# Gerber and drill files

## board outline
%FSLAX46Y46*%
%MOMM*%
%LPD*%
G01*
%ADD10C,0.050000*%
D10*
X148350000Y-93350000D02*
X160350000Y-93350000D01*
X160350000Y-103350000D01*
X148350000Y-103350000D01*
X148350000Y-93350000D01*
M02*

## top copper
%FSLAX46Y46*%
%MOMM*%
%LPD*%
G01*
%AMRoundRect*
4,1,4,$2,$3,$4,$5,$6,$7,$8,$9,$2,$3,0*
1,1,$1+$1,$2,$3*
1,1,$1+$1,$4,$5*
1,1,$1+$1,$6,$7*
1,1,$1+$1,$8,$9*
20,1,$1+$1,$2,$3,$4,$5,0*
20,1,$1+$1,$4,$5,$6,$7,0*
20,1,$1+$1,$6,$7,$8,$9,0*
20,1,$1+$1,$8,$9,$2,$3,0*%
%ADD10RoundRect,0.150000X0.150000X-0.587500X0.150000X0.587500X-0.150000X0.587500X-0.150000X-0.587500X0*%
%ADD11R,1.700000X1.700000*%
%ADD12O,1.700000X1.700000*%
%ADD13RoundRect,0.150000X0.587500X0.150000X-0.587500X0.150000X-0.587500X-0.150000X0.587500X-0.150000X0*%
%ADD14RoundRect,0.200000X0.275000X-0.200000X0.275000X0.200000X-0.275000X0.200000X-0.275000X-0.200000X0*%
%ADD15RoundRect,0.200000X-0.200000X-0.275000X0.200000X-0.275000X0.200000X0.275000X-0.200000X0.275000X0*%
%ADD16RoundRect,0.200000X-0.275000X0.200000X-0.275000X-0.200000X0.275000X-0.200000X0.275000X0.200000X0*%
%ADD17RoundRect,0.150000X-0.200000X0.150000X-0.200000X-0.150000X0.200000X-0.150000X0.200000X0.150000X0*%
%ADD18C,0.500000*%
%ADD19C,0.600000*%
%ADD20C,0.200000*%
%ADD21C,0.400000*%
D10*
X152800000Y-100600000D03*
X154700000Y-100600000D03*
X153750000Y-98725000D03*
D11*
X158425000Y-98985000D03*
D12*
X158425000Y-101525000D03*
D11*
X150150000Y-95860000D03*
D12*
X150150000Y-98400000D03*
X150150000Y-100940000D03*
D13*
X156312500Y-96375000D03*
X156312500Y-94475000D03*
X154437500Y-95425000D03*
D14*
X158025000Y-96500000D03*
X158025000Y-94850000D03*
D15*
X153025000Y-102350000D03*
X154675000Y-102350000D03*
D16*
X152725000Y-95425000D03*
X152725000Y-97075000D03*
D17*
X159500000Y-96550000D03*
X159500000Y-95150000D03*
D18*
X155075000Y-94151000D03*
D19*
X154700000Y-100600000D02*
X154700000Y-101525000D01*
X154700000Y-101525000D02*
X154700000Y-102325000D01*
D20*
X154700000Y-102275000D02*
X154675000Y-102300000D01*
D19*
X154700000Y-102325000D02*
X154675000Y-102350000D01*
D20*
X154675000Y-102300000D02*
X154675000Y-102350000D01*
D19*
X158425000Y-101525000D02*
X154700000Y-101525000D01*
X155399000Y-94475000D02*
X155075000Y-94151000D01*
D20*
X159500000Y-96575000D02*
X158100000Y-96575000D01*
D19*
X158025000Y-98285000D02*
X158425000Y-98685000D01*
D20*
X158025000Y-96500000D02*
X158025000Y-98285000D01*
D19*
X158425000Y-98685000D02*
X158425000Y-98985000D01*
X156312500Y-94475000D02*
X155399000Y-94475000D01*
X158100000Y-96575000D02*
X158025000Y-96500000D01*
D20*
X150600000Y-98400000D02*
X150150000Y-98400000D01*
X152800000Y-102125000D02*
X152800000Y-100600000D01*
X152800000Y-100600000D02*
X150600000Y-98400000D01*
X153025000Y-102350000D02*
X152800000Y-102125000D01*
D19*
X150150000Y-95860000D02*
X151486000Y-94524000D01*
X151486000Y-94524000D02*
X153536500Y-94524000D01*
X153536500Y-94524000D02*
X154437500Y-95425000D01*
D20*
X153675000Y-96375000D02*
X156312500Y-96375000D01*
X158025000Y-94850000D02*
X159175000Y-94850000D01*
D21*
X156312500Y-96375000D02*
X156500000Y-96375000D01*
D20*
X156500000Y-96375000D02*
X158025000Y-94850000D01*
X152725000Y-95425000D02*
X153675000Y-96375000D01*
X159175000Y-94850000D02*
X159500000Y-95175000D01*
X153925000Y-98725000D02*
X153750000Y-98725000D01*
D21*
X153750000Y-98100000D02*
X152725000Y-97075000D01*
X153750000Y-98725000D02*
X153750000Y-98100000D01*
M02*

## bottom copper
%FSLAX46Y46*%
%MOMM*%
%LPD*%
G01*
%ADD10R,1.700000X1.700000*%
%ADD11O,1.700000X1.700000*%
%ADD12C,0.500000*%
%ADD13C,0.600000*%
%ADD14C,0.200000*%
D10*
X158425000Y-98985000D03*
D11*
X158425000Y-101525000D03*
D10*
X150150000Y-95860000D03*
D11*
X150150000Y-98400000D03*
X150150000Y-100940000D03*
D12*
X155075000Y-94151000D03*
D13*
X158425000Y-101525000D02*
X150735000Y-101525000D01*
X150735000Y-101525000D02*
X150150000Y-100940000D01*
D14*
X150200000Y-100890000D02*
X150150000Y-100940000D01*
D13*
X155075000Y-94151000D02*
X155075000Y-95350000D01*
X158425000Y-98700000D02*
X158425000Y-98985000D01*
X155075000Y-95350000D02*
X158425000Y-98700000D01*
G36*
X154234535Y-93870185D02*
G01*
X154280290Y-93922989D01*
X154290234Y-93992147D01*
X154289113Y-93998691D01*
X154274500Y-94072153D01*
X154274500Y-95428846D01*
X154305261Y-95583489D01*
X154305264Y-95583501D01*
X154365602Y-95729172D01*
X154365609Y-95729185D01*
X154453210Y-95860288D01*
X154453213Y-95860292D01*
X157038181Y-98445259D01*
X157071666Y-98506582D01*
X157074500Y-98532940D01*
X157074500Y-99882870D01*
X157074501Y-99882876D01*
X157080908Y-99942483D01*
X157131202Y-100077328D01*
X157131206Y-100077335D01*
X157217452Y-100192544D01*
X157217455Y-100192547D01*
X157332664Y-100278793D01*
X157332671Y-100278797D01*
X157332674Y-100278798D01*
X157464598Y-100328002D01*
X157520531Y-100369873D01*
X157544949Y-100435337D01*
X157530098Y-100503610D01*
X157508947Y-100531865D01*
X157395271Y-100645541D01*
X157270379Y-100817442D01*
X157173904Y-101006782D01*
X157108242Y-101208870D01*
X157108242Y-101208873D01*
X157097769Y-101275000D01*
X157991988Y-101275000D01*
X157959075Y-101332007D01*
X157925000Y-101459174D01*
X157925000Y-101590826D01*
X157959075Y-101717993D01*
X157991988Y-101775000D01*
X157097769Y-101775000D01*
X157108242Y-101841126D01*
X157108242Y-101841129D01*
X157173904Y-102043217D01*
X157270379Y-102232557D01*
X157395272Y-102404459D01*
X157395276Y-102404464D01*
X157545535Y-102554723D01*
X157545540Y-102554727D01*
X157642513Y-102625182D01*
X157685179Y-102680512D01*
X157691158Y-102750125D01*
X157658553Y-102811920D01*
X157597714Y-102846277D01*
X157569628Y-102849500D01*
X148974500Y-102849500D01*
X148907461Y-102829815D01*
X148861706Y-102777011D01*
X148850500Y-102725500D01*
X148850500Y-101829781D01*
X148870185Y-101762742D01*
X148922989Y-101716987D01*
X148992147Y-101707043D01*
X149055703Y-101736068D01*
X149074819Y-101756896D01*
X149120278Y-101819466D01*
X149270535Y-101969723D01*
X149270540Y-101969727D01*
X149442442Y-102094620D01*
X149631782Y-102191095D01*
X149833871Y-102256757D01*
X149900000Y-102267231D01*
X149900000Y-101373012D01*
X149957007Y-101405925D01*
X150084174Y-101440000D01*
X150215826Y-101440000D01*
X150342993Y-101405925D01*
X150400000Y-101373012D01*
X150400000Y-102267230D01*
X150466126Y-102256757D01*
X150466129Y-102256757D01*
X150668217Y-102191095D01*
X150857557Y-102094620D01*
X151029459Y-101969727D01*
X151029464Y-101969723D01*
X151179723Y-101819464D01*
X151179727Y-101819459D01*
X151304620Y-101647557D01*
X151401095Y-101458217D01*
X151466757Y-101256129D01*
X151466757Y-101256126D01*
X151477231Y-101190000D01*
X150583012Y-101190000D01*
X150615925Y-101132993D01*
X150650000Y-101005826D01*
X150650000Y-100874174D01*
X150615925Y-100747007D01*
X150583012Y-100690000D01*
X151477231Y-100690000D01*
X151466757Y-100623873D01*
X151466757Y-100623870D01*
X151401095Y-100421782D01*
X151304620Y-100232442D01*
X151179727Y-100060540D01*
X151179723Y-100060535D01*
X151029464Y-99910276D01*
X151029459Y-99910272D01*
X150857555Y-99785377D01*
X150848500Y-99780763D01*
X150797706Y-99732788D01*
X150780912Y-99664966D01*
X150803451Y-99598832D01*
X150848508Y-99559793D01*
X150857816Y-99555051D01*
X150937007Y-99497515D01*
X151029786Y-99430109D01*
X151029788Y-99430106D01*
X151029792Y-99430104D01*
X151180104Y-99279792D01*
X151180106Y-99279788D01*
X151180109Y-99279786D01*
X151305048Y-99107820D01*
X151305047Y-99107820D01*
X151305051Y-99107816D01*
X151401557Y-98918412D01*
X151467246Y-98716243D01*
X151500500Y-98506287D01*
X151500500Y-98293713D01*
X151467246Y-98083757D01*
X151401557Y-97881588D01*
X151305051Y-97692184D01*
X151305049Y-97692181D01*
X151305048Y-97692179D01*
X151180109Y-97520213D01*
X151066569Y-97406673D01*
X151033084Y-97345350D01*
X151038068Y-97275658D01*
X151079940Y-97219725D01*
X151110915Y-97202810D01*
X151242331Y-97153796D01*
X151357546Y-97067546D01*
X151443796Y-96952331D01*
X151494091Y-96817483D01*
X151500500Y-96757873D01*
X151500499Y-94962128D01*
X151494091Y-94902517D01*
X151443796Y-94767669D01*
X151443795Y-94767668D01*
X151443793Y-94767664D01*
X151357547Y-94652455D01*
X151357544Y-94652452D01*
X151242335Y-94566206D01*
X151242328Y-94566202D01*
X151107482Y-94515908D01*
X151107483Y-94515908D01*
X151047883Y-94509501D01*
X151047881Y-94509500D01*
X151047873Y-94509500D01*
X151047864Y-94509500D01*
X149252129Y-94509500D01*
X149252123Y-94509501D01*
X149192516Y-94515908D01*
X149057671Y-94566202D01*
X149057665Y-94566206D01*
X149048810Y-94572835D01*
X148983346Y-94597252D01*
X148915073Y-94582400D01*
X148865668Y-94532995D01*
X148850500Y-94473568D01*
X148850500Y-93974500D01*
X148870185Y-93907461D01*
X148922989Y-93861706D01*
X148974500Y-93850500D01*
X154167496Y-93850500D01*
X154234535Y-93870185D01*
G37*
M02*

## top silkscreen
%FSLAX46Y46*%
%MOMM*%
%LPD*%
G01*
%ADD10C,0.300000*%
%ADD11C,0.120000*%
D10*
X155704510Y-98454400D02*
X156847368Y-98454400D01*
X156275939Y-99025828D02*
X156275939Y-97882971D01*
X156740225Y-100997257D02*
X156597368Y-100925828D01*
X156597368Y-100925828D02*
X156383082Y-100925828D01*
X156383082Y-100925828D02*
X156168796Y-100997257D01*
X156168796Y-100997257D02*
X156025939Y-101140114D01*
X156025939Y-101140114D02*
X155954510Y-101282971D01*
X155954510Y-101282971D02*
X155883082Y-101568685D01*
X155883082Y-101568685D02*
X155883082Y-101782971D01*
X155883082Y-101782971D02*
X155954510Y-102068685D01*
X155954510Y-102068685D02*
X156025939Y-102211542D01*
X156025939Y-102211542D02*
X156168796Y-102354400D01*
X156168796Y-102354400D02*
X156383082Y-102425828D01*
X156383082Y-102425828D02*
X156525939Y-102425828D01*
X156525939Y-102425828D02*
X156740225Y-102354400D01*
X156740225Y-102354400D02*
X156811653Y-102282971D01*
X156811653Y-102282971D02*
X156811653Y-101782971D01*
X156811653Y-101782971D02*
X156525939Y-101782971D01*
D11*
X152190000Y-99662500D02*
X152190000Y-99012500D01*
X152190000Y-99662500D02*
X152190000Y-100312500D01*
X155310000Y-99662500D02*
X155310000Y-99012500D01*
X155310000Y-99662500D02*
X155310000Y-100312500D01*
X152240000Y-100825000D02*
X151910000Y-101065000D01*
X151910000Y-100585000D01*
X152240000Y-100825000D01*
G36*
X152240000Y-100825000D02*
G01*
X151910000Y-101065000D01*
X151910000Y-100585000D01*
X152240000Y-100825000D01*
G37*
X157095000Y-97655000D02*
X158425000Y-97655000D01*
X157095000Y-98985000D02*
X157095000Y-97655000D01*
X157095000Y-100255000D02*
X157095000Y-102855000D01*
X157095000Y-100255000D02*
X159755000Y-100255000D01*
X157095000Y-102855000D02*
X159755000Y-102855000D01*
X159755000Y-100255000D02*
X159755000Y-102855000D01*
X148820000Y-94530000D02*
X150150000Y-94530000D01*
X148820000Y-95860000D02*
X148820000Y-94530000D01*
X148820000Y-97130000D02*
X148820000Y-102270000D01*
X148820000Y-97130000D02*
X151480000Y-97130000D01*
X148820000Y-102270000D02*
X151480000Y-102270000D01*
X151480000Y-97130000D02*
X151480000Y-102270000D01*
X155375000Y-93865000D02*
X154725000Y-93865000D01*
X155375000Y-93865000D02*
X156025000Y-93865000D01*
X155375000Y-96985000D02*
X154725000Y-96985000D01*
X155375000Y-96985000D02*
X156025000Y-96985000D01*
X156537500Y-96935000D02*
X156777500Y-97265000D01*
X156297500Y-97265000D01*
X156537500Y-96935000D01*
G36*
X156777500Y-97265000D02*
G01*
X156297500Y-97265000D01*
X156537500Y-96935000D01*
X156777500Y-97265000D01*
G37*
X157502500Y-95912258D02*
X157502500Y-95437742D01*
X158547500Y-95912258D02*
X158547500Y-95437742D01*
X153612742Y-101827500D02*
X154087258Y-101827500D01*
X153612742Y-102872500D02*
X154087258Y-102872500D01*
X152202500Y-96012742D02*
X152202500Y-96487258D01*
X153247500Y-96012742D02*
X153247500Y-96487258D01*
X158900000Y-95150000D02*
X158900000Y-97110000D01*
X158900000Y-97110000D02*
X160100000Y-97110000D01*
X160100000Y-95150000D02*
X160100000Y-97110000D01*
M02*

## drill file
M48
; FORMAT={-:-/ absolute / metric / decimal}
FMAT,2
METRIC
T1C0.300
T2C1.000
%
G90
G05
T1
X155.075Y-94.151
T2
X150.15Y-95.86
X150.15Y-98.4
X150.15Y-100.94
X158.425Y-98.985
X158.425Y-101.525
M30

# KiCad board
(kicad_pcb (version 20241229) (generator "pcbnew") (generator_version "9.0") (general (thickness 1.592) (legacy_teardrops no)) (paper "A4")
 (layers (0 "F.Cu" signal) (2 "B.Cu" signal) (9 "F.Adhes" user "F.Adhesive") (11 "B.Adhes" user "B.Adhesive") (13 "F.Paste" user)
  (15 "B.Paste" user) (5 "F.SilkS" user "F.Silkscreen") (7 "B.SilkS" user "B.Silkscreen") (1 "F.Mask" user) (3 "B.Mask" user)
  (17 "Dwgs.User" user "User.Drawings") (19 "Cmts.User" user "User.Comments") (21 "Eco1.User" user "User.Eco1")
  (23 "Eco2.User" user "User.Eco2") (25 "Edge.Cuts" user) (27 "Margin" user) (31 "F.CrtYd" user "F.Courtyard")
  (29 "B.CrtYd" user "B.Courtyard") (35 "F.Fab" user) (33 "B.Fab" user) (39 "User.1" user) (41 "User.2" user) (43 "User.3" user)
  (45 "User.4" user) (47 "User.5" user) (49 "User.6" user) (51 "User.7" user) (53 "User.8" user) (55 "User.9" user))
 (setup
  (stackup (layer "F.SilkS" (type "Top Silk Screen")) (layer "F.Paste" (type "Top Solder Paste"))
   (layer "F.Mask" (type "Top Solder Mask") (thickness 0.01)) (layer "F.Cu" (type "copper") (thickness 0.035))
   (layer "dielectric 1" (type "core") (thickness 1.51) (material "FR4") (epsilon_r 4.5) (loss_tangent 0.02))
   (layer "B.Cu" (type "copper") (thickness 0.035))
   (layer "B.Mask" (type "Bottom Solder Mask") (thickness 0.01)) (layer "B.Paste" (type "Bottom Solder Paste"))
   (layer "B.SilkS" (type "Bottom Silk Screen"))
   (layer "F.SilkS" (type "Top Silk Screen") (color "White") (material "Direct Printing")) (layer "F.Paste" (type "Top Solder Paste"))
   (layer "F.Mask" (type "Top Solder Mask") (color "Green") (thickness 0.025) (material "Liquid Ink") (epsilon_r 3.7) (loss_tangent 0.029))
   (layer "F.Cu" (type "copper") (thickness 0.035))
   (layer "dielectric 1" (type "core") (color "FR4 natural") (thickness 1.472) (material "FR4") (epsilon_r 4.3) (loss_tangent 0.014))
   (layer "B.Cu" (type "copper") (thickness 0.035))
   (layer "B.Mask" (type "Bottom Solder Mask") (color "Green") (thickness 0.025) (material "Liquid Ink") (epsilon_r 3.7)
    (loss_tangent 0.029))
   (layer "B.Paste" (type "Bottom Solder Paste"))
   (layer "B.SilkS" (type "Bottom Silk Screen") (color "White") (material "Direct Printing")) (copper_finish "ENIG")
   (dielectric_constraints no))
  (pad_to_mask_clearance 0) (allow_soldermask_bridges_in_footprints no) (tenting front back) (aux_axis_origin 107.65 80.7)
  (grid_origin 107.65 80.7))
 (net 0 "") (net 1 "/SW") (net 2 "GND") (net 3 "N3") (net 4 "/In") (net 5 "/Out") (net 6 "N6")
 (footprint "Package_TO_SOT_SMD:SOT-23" (layer "F.Cu") (at 153.75 99.6625 90)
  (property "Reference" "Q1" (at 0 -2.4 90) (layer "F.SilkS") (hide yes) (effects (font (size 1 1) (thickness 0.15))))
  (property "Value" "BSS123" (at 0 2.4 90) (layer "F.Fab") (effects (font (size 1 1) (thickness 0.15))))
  (fp_line (start 0 -1.56) (end 0.65 -1.56) (stroke (width 0.12) (type solid)) (layer "F.SilkS"))
  (fp_line (start 0 -1.56) (end -0.65 -1.56) (stroke (width 0.12) (type solid)) (layer "F.SilkS"))
  (fp_line (start 0 1.56) (end 0.65 1.56) (stroke (width 0.12) (type solid)) (layer "F.SilkS"))
  (fp_line (start 0 1.56) (end -0.65 1.56) (stroke (width 0.12) (type solid)) (layer "F.SilkS"))
  (fp_poly
   (pts (xy -1.1625 -1.51) (xy -1.4025 -1.84) (xy -0.9225 -1.84) (xy -1.1625 -1.51)) (stroke (width 0.12) (type solid)) (fill yes)
   (layer "F.SilkS"))
  (pad "1" smd roundrect (at -0.9375 -0.95 90) (size 1.475 0.6) (layers "F.Cu" "F.Mask" "F.Paste") (roundrect_rratio 0.25) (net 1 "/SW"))
  (pad "2" smd roundrect (at -0.9375 0.95 90) (size 1.475 0.6) (layers "F.Cu" "F.Mask" "F.Paste") (roundrect_rratio 0.25) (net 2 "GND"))
  (pad "3" smd roundrect (at 0.9375 0 90) (size 1.475 0.6) (layers "F.Cu" "F.Mask" "F.Paste") (roundrect_rratio 0.25) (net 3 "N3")))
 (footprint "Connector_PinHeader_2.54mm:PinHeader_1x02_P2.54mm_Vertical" (layer "F.Cu") (at 158.425 98.985)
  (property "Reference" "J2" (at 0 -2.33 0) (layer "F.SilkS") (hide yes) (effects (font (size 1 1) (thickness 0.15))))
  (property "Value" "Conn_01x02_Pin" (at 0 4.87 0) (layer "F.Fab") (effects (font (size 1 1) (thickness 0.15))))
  (fp_line (start -1.33 -1.33) (end 0 -1.33) (stroke (width 0.12) (type solid)) (layer "F.SilkS"))
  (fp_line (start -1.33 0) (end -1.33 -1.33) (stroke (width 0.12) (type solid)) (layer "F.SilkS"))
  (fp_line (start -1.33 1.27) (end -1.33 3.87) (stroke (width 0.12) (type solid)) (layer "F.SilkS"))
  (fp_line (start -1.33 1.27) (end 1.33 1.27) (stroke (width 0.12) (type solid)) (layer "F.SilkS"))
  (fp_line (start -1.33 3.87) (end 1.33 3.87) (stroke (width 0.12) (type solid)) (layer "F.SilkS"))
  (fp_line (start 1.33 1.27) (end 1.33 3.87) (stroke (width 0.12) (type solid)) (layer "F.SilkS"))
  (pad "1" thru_hole rect (at 0 0) (size 1.7 1.7) (drill 1) (layers "*.Cu" "*.Mask") (remove_unused_layers no) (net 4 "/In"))
  (pad "2" thru_hole oval (at 0 2.54) (size 1.7 1.7) (drill 1) (layers "*.Cu" "*.Mask") (remove_unused_layers no) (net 2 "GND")))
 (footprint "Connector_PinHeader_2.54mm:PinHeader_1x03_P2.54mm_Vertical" (layer "F.Cu") (at 150.15 95.86)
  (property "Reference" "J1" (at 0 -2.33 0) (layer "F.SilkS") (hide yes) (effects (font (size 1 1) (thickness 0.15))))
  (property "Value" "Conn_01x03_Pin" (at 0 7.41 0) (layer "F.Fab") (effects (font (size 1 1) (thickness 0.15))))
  (fp_line (start -1.33 -1.33) (end 0 -1.33) (stroke (width 0.12) (type solid)) (layer "F.SilkS"))
  (fp_line (start -1.33 0) (end -1.33 -1.33) (stroke (width 0.12) (type solid)) (layer "F.SilkS"))
  (fp_line (start -1.33 1.27) (end -1.33 6.41) (stroke (width 0.12) (type solid)) (layer "F.SilkS"))
  (fp_line (start -1.33 1.27) (end 1.33 1.27) (stroke (width 0.12) (type solid)) (layer "F.SilkS"))
  (fp_line (start -1.33 6.41) (end 1.33 6.41) (stroke (width 0.12) (type solid)) (layer "F.SilkS"))
  (fp_line (start 1.33 1.27) (end 1.33 6.41) (stroke (width 0.12) (type solid)) (layer "F.SilkS"))
  (pad "1" thru_hole rect (at 0 0) (size 1.7 1.7) (drill 1) (layers "*.Cu" "*.Mask") (remove_unused_layers no) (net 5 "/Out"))
  (pad "2" thru_hole oval (at 0 2.54) (size 1.7 1.7) (drill 1) (layers "*.Cu" "*.Mask") (remove_unused_layers no) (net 1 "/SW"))
  (pad "3" thru_hole oval (at 0 5.08) (size 1.7 1.7) (drill 1) (layers "*.Cu" "*.Mask") (remove_unused_layers no) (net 2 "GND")))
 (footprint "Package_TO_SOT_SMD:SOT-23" (layer "F.Cu") (at 155.375 95.425 180)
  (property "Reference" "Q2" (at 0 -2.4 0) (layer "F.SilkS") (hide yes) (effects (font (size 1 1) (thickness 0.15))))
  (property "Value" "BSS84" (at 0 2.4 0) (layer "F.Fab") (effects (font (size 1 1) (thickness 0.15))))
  (fp_line (start 0 1.56) (end 0.65 1.56) (stroke (width 0.12) (type solid)) (layer "F.SilkS"))
  (fp_line (start 0 1.56) (end -0.65 1.56) (stroke (width 0.12) (type solid)) (layer "F.SilkS"))
  (fp_line (start 0 -1.56) (end 0.65 -1.56) (stroke (width 0.12) (type solid)) (layer "F.SilkS"))
  (fp_line (start 0 -1.56) (end -0.65 -1.56) (stroke (width 0.12) (type solid)) (layer "F.SilkS"))
  (fp_poly
   (pts (xy -1.1625 -1.51) (xy -1.4025 -1.84) (xy -0.9225 -1.84) (xy -1.1625 -1.51)) (stroke (width 0.12) (type solid)) (fill yes)
   (layer "F.SilkS"))
  (pad "1" smd roundrect (at -0.9375 -0.95 180) (size 1.475 0.6) (layers "F.Cu" "F.Mask" "F.Paste") (roundrect_rratio 0.25) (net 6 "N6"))
  (pad "2" smd roundrect (at -0.9375 0.95 180) (size 1.475 0.6) (layers "F.Cu" "F.Mask" "F.Paste") (roundrect_rratio 0.25) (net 4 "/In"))
  (pad "3" smd roundrect (at 0.9375 0 180) (size 1.475 0.6) (layers "F.Cu" "F.Mask" "F.Paste") (roundrect_rratio 0.25) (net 5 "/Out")))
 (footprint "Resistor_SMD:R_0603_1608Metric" (layer "F.Cu") (at 158.025 95.675 90)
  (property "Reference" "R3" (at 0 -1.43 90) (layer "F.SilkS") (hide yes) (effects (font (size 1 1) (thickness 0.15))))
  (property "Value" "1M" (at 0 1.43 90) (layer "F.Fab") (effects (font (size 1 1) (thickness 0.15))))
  (fp_line (start -0.237258 -0.5225) (end 0.237258 -0.5225) (stroke (width 0.12) (type solid)) (layer "F.SilkS"))
  (fp_line (start -0.237258 0.5225) (end 0.237258 0.5225) (stroke (width 0.12) (type solid)) (layer "F.SilkS"))
  (pad "1" smd roundrect (at -0.825 0 90) (size 0.8 0.95) (layers "F.Cu" "F.Mask" "F.Paste") (roundrect_rratio 0.25) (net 4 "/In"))
  (pad "2" smd roundrect (at 0.825 0 90) (size 0.8 0.95) (layers "F.Cu" "F.Mask" "F.Paste") (roundrect_rratio 0.25) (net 6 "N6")))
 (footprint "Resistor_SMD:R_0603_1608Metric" (layer "F.Cu") (at 153.85 102.35)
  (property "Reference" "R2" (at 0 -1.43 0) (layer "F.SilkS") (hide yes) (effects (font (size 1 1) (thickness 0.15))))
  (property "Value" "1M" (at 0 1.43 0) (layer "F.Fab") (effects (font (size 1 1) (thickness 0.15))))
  (fp_line (start -0.237258 -0.5225) (end 0.237258 -0.5225) (stroke (width 0.12) (type solid)) (layer "F.SilkS"))
  (fp_line (start -0.237258 0.5225) (end 0.237258 0.5225) (stroke (width 0.12) (type solid)) (layer "F.SilkS"))
  (pad "1" smd roundrect (at -0.825 0) (size 0.8 0.95) (layers "F.Cu" "F.Mask" "F.Paste") (roundrect_rratio 0.25) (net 1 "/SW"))
  (pad "2" smd roundrect (at 0.825 0) (size 0.8 0.95) (layers "F.Cu" "F.Mask" "F.Paste") (roundrect_rratio 0.25) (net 2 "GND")))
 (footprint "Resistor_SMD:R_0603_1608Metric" (layer "F.Cu") (at 152.725 96.25 -90)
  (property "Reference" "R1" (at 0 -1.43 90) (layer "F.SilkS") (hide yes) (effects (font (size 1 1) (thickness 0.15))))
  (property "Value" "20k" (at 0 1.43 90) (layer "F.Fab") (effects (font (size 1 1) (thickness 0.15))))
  (fp_line (start -0.237258 0.5225) (end 0.237258 0.5225) (stroke (width 0.12) (type solid)) (layer "F.SilkS"))
  (fp_line (start -0.237258 -0.5225) (end 0.237258 -0.5225) (stroke (width 0.12) (type solid)) (layer "F.SilkS"))
  (pad "1" smd roundrect (at -0.825 0 270) (size 0.8 0.95) (layers "F.Cu" "F.Mask" "F.Paste") (roundrect_rratio 0.25) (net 6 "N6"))
  (pad "2" smd roundrect (at 0.825 0 270) (size 0.8 0.95) (layers "F.Cu" "F.Mask" "F.Paste") (roundrect_rratio 0.25) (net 3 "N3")))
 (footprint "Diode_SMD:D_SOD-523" (layer "F.Cu") (at 159.5 95.85 90)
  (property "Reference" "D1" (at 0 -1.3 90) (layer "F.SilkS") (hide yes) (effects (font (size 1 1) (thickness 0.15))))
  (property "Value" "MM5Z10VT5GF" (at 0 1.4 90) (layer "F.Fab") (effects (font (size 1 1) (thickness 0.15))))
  (fp_line (start 0.7 -0.6) (end -1.26 -0.6) (stroke (width 0.12) (type solid)) (layer "F.SilkS"))
  (fp_line (start -1.26 -0.6) (end -1.26 0.6) (stroke (width 0.12) (type solid)) (layer "F.SilkS"))
  (fp_line (start 0.7 0.6) (end -1.26 0.6) (stroke (width 0.12) (type solid)) (layer "F.SilkS"))
  (pad "1" smd roundrect (at -0.7 0 270) (size 0.6 0.7) (layers "F.Cu" "F.Mask" "F.Paste") (roundrect_rratio 0.25) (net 4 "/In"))
  (pad "2" smd roundrect (at 0.7 0 270) (size 0.6 0.7) (layers "F.Cu" "F.Mask" "F.Paste") (roundrect_rratio 0.25) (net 6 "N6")))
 (gr_rect (start 148.35 93.35) (end 160.35 103.35) (stroke (width 0.05) (type solid)) (fill no) (layer "Edge.Cuts"))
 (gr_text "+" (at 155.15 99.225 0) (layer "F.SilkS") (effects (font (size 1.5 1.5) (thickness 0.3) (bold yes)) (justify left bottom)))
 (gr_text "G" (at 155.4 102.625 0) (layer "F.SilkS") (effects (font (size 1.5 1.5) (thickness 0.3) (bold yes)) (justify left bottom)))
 (segment (start 154.7 100.6) (end 154.7 101.525) (width 0.6) (layer "F.Cu") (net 2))
 (segment (start 154.7 101.525) (end 154.7 102.325) (width 0.6) (layer "F.Cu") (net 2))
 (segment (start 154.7 102.275) (end 154.675 102.3) (width 0.2) (layer "F.Cu") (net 2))
 (segment (start 154.7 102.325) (end 154.675 102.35) (width 0.6) (layer "F.Cu") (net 2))
 (segment (start 154.675 102.3) (end 154.675 102.35) (width 0.2) (layer "F.Cu") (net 2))
 (segment (start 158.425 101.525) (end 154.7 101.525) (width 0.6) (layer "F.Cu") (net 2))
 (segment (start 158.425 101.525) (end 150.735 101.525) (width 0.6) (layer "B.Cu") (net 2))
 (segment (start 150.735 101.525) (end 150.15 100.94) (width 0.6) (layer "B.Cu") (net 2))
 (segment (start 150.2 100.89) (end 150.15 100.94) (width 0.2) (layer "B.Cu") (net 2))
 (segment (start 155.399 94.475) (end 155.075 94.151) (width 0.6) (layer "F.Cu") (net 4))
 (segment (start 159.5 96.575) (end 158.1 96.575) (width 0.2) (layer "F.Cu") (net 4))
 (segment (start 158.025 98.285) (end 158.425 98.685) (width 0.6) (layer "F.Cu") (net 4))
 (segment (start 158.025 96.5) (end 158.025 98.285) (width 0.2) (layer "F.Cu") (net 4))
 (segment (start 158.425 98.685) (end 158.425 98.985) (width 0.6) (layer "F.Cu") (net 4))
 (segment (start 156.3125 94.475) (end 155.399 94.475) (width 0.6) (layer "F.Cu") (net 4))
 (segment (start 158.1 96.575) (end 158.025 96.5) (width 0.6) (layer "F.Cu") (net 4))
 (via (at 155.075 94.151) (size 0.5) (drill 0.3) (layers "F.Cu" "B.Cu") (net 4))
 (segment (start 155.075 94.151) (end 155.075 95.35) (width 0.6) (layer "B.Cu") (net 4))
 (segment (start 158.425 98.7) (end 158.425 98.985) (width 0.6) (layer "B.Cu") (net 4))
 (segment (start 155.075 95.35) (end 158.425 98.7) (width 0.6) (layer "B.Cu") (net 4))
 (segment (start 150.6 98.4) (end 150.15 98.4) (width 0.2) (layer "F.Cu") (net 1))
 (segment (start 152.8 102.125) (end 152.8 100.6) (width 0.2) (layer "F.Cu") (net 1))
 (segment (start 152.8 100.6) (end 150.6 98.4) (width 0.2) (layer "F.Cu") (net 1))
 (segment (start 153.025 102.35) (end 152.8 102.125) (width 0.2) (layer "F.Cu") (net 1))
 (segment (start 150.15 95.86) (end 151.486 94.524) (width 0.6) (layer "F.Cu") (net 5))
 (segment (start 151.486 94.524) (end 153.5365 94.524) (width 0.6) (layer "F.Cu") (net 5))
 (segment (start 153.5365 94.524) (end 154.4375 95.425) (width 0.6) (layer "F.Cu") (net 5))
 (segment (start 153.675 96.375) (end 156.3125 96.375) (width 0.2) (layer "F.Cu") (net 6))
 (segment (start 158.025 94.85) (end 159.175 94.85) (width 0.2) (layer "F.Cu") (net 6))
 (segment (start 156.3125 96.375) (end 156.5 96.375) (width 0.4) (layer "F.Cu") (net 6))
 (segment (start 156.5 96.375) (end 158.025 94.85) (width 0.2) (layer "F.Cu") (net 6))
 (segment (start 152.725 95.425) (end 153.675 96.375) (width 0.2) (layer "F.Cu") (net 6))
 (segment (start 159.175 94.85) (end 159.5 95.175) (width 0.2) (layer "F.Cu") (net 6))
 (segment (start 153.925 98.725) (end 153.75 98.725) (width 0.2) (layer "F.Cu") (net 3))
 (segment (start 153.75 98.1) (end 152.725 97.075) (width 0.4) (layer "F.Cu") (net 3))
 (segment (start 153.75 98.725) (end 153.75 98.1) (width 0.4) (layer "F.Cu") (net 3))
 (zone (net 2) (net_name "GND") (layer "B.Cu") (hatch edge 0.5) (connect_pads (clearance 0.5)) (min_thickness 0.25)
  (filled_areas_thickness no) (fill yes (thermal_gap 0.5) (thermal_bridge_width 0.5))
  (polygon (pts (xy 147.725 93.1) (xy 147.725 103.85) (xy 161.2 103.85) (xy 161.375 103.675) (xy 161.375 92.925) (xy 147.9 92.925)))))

